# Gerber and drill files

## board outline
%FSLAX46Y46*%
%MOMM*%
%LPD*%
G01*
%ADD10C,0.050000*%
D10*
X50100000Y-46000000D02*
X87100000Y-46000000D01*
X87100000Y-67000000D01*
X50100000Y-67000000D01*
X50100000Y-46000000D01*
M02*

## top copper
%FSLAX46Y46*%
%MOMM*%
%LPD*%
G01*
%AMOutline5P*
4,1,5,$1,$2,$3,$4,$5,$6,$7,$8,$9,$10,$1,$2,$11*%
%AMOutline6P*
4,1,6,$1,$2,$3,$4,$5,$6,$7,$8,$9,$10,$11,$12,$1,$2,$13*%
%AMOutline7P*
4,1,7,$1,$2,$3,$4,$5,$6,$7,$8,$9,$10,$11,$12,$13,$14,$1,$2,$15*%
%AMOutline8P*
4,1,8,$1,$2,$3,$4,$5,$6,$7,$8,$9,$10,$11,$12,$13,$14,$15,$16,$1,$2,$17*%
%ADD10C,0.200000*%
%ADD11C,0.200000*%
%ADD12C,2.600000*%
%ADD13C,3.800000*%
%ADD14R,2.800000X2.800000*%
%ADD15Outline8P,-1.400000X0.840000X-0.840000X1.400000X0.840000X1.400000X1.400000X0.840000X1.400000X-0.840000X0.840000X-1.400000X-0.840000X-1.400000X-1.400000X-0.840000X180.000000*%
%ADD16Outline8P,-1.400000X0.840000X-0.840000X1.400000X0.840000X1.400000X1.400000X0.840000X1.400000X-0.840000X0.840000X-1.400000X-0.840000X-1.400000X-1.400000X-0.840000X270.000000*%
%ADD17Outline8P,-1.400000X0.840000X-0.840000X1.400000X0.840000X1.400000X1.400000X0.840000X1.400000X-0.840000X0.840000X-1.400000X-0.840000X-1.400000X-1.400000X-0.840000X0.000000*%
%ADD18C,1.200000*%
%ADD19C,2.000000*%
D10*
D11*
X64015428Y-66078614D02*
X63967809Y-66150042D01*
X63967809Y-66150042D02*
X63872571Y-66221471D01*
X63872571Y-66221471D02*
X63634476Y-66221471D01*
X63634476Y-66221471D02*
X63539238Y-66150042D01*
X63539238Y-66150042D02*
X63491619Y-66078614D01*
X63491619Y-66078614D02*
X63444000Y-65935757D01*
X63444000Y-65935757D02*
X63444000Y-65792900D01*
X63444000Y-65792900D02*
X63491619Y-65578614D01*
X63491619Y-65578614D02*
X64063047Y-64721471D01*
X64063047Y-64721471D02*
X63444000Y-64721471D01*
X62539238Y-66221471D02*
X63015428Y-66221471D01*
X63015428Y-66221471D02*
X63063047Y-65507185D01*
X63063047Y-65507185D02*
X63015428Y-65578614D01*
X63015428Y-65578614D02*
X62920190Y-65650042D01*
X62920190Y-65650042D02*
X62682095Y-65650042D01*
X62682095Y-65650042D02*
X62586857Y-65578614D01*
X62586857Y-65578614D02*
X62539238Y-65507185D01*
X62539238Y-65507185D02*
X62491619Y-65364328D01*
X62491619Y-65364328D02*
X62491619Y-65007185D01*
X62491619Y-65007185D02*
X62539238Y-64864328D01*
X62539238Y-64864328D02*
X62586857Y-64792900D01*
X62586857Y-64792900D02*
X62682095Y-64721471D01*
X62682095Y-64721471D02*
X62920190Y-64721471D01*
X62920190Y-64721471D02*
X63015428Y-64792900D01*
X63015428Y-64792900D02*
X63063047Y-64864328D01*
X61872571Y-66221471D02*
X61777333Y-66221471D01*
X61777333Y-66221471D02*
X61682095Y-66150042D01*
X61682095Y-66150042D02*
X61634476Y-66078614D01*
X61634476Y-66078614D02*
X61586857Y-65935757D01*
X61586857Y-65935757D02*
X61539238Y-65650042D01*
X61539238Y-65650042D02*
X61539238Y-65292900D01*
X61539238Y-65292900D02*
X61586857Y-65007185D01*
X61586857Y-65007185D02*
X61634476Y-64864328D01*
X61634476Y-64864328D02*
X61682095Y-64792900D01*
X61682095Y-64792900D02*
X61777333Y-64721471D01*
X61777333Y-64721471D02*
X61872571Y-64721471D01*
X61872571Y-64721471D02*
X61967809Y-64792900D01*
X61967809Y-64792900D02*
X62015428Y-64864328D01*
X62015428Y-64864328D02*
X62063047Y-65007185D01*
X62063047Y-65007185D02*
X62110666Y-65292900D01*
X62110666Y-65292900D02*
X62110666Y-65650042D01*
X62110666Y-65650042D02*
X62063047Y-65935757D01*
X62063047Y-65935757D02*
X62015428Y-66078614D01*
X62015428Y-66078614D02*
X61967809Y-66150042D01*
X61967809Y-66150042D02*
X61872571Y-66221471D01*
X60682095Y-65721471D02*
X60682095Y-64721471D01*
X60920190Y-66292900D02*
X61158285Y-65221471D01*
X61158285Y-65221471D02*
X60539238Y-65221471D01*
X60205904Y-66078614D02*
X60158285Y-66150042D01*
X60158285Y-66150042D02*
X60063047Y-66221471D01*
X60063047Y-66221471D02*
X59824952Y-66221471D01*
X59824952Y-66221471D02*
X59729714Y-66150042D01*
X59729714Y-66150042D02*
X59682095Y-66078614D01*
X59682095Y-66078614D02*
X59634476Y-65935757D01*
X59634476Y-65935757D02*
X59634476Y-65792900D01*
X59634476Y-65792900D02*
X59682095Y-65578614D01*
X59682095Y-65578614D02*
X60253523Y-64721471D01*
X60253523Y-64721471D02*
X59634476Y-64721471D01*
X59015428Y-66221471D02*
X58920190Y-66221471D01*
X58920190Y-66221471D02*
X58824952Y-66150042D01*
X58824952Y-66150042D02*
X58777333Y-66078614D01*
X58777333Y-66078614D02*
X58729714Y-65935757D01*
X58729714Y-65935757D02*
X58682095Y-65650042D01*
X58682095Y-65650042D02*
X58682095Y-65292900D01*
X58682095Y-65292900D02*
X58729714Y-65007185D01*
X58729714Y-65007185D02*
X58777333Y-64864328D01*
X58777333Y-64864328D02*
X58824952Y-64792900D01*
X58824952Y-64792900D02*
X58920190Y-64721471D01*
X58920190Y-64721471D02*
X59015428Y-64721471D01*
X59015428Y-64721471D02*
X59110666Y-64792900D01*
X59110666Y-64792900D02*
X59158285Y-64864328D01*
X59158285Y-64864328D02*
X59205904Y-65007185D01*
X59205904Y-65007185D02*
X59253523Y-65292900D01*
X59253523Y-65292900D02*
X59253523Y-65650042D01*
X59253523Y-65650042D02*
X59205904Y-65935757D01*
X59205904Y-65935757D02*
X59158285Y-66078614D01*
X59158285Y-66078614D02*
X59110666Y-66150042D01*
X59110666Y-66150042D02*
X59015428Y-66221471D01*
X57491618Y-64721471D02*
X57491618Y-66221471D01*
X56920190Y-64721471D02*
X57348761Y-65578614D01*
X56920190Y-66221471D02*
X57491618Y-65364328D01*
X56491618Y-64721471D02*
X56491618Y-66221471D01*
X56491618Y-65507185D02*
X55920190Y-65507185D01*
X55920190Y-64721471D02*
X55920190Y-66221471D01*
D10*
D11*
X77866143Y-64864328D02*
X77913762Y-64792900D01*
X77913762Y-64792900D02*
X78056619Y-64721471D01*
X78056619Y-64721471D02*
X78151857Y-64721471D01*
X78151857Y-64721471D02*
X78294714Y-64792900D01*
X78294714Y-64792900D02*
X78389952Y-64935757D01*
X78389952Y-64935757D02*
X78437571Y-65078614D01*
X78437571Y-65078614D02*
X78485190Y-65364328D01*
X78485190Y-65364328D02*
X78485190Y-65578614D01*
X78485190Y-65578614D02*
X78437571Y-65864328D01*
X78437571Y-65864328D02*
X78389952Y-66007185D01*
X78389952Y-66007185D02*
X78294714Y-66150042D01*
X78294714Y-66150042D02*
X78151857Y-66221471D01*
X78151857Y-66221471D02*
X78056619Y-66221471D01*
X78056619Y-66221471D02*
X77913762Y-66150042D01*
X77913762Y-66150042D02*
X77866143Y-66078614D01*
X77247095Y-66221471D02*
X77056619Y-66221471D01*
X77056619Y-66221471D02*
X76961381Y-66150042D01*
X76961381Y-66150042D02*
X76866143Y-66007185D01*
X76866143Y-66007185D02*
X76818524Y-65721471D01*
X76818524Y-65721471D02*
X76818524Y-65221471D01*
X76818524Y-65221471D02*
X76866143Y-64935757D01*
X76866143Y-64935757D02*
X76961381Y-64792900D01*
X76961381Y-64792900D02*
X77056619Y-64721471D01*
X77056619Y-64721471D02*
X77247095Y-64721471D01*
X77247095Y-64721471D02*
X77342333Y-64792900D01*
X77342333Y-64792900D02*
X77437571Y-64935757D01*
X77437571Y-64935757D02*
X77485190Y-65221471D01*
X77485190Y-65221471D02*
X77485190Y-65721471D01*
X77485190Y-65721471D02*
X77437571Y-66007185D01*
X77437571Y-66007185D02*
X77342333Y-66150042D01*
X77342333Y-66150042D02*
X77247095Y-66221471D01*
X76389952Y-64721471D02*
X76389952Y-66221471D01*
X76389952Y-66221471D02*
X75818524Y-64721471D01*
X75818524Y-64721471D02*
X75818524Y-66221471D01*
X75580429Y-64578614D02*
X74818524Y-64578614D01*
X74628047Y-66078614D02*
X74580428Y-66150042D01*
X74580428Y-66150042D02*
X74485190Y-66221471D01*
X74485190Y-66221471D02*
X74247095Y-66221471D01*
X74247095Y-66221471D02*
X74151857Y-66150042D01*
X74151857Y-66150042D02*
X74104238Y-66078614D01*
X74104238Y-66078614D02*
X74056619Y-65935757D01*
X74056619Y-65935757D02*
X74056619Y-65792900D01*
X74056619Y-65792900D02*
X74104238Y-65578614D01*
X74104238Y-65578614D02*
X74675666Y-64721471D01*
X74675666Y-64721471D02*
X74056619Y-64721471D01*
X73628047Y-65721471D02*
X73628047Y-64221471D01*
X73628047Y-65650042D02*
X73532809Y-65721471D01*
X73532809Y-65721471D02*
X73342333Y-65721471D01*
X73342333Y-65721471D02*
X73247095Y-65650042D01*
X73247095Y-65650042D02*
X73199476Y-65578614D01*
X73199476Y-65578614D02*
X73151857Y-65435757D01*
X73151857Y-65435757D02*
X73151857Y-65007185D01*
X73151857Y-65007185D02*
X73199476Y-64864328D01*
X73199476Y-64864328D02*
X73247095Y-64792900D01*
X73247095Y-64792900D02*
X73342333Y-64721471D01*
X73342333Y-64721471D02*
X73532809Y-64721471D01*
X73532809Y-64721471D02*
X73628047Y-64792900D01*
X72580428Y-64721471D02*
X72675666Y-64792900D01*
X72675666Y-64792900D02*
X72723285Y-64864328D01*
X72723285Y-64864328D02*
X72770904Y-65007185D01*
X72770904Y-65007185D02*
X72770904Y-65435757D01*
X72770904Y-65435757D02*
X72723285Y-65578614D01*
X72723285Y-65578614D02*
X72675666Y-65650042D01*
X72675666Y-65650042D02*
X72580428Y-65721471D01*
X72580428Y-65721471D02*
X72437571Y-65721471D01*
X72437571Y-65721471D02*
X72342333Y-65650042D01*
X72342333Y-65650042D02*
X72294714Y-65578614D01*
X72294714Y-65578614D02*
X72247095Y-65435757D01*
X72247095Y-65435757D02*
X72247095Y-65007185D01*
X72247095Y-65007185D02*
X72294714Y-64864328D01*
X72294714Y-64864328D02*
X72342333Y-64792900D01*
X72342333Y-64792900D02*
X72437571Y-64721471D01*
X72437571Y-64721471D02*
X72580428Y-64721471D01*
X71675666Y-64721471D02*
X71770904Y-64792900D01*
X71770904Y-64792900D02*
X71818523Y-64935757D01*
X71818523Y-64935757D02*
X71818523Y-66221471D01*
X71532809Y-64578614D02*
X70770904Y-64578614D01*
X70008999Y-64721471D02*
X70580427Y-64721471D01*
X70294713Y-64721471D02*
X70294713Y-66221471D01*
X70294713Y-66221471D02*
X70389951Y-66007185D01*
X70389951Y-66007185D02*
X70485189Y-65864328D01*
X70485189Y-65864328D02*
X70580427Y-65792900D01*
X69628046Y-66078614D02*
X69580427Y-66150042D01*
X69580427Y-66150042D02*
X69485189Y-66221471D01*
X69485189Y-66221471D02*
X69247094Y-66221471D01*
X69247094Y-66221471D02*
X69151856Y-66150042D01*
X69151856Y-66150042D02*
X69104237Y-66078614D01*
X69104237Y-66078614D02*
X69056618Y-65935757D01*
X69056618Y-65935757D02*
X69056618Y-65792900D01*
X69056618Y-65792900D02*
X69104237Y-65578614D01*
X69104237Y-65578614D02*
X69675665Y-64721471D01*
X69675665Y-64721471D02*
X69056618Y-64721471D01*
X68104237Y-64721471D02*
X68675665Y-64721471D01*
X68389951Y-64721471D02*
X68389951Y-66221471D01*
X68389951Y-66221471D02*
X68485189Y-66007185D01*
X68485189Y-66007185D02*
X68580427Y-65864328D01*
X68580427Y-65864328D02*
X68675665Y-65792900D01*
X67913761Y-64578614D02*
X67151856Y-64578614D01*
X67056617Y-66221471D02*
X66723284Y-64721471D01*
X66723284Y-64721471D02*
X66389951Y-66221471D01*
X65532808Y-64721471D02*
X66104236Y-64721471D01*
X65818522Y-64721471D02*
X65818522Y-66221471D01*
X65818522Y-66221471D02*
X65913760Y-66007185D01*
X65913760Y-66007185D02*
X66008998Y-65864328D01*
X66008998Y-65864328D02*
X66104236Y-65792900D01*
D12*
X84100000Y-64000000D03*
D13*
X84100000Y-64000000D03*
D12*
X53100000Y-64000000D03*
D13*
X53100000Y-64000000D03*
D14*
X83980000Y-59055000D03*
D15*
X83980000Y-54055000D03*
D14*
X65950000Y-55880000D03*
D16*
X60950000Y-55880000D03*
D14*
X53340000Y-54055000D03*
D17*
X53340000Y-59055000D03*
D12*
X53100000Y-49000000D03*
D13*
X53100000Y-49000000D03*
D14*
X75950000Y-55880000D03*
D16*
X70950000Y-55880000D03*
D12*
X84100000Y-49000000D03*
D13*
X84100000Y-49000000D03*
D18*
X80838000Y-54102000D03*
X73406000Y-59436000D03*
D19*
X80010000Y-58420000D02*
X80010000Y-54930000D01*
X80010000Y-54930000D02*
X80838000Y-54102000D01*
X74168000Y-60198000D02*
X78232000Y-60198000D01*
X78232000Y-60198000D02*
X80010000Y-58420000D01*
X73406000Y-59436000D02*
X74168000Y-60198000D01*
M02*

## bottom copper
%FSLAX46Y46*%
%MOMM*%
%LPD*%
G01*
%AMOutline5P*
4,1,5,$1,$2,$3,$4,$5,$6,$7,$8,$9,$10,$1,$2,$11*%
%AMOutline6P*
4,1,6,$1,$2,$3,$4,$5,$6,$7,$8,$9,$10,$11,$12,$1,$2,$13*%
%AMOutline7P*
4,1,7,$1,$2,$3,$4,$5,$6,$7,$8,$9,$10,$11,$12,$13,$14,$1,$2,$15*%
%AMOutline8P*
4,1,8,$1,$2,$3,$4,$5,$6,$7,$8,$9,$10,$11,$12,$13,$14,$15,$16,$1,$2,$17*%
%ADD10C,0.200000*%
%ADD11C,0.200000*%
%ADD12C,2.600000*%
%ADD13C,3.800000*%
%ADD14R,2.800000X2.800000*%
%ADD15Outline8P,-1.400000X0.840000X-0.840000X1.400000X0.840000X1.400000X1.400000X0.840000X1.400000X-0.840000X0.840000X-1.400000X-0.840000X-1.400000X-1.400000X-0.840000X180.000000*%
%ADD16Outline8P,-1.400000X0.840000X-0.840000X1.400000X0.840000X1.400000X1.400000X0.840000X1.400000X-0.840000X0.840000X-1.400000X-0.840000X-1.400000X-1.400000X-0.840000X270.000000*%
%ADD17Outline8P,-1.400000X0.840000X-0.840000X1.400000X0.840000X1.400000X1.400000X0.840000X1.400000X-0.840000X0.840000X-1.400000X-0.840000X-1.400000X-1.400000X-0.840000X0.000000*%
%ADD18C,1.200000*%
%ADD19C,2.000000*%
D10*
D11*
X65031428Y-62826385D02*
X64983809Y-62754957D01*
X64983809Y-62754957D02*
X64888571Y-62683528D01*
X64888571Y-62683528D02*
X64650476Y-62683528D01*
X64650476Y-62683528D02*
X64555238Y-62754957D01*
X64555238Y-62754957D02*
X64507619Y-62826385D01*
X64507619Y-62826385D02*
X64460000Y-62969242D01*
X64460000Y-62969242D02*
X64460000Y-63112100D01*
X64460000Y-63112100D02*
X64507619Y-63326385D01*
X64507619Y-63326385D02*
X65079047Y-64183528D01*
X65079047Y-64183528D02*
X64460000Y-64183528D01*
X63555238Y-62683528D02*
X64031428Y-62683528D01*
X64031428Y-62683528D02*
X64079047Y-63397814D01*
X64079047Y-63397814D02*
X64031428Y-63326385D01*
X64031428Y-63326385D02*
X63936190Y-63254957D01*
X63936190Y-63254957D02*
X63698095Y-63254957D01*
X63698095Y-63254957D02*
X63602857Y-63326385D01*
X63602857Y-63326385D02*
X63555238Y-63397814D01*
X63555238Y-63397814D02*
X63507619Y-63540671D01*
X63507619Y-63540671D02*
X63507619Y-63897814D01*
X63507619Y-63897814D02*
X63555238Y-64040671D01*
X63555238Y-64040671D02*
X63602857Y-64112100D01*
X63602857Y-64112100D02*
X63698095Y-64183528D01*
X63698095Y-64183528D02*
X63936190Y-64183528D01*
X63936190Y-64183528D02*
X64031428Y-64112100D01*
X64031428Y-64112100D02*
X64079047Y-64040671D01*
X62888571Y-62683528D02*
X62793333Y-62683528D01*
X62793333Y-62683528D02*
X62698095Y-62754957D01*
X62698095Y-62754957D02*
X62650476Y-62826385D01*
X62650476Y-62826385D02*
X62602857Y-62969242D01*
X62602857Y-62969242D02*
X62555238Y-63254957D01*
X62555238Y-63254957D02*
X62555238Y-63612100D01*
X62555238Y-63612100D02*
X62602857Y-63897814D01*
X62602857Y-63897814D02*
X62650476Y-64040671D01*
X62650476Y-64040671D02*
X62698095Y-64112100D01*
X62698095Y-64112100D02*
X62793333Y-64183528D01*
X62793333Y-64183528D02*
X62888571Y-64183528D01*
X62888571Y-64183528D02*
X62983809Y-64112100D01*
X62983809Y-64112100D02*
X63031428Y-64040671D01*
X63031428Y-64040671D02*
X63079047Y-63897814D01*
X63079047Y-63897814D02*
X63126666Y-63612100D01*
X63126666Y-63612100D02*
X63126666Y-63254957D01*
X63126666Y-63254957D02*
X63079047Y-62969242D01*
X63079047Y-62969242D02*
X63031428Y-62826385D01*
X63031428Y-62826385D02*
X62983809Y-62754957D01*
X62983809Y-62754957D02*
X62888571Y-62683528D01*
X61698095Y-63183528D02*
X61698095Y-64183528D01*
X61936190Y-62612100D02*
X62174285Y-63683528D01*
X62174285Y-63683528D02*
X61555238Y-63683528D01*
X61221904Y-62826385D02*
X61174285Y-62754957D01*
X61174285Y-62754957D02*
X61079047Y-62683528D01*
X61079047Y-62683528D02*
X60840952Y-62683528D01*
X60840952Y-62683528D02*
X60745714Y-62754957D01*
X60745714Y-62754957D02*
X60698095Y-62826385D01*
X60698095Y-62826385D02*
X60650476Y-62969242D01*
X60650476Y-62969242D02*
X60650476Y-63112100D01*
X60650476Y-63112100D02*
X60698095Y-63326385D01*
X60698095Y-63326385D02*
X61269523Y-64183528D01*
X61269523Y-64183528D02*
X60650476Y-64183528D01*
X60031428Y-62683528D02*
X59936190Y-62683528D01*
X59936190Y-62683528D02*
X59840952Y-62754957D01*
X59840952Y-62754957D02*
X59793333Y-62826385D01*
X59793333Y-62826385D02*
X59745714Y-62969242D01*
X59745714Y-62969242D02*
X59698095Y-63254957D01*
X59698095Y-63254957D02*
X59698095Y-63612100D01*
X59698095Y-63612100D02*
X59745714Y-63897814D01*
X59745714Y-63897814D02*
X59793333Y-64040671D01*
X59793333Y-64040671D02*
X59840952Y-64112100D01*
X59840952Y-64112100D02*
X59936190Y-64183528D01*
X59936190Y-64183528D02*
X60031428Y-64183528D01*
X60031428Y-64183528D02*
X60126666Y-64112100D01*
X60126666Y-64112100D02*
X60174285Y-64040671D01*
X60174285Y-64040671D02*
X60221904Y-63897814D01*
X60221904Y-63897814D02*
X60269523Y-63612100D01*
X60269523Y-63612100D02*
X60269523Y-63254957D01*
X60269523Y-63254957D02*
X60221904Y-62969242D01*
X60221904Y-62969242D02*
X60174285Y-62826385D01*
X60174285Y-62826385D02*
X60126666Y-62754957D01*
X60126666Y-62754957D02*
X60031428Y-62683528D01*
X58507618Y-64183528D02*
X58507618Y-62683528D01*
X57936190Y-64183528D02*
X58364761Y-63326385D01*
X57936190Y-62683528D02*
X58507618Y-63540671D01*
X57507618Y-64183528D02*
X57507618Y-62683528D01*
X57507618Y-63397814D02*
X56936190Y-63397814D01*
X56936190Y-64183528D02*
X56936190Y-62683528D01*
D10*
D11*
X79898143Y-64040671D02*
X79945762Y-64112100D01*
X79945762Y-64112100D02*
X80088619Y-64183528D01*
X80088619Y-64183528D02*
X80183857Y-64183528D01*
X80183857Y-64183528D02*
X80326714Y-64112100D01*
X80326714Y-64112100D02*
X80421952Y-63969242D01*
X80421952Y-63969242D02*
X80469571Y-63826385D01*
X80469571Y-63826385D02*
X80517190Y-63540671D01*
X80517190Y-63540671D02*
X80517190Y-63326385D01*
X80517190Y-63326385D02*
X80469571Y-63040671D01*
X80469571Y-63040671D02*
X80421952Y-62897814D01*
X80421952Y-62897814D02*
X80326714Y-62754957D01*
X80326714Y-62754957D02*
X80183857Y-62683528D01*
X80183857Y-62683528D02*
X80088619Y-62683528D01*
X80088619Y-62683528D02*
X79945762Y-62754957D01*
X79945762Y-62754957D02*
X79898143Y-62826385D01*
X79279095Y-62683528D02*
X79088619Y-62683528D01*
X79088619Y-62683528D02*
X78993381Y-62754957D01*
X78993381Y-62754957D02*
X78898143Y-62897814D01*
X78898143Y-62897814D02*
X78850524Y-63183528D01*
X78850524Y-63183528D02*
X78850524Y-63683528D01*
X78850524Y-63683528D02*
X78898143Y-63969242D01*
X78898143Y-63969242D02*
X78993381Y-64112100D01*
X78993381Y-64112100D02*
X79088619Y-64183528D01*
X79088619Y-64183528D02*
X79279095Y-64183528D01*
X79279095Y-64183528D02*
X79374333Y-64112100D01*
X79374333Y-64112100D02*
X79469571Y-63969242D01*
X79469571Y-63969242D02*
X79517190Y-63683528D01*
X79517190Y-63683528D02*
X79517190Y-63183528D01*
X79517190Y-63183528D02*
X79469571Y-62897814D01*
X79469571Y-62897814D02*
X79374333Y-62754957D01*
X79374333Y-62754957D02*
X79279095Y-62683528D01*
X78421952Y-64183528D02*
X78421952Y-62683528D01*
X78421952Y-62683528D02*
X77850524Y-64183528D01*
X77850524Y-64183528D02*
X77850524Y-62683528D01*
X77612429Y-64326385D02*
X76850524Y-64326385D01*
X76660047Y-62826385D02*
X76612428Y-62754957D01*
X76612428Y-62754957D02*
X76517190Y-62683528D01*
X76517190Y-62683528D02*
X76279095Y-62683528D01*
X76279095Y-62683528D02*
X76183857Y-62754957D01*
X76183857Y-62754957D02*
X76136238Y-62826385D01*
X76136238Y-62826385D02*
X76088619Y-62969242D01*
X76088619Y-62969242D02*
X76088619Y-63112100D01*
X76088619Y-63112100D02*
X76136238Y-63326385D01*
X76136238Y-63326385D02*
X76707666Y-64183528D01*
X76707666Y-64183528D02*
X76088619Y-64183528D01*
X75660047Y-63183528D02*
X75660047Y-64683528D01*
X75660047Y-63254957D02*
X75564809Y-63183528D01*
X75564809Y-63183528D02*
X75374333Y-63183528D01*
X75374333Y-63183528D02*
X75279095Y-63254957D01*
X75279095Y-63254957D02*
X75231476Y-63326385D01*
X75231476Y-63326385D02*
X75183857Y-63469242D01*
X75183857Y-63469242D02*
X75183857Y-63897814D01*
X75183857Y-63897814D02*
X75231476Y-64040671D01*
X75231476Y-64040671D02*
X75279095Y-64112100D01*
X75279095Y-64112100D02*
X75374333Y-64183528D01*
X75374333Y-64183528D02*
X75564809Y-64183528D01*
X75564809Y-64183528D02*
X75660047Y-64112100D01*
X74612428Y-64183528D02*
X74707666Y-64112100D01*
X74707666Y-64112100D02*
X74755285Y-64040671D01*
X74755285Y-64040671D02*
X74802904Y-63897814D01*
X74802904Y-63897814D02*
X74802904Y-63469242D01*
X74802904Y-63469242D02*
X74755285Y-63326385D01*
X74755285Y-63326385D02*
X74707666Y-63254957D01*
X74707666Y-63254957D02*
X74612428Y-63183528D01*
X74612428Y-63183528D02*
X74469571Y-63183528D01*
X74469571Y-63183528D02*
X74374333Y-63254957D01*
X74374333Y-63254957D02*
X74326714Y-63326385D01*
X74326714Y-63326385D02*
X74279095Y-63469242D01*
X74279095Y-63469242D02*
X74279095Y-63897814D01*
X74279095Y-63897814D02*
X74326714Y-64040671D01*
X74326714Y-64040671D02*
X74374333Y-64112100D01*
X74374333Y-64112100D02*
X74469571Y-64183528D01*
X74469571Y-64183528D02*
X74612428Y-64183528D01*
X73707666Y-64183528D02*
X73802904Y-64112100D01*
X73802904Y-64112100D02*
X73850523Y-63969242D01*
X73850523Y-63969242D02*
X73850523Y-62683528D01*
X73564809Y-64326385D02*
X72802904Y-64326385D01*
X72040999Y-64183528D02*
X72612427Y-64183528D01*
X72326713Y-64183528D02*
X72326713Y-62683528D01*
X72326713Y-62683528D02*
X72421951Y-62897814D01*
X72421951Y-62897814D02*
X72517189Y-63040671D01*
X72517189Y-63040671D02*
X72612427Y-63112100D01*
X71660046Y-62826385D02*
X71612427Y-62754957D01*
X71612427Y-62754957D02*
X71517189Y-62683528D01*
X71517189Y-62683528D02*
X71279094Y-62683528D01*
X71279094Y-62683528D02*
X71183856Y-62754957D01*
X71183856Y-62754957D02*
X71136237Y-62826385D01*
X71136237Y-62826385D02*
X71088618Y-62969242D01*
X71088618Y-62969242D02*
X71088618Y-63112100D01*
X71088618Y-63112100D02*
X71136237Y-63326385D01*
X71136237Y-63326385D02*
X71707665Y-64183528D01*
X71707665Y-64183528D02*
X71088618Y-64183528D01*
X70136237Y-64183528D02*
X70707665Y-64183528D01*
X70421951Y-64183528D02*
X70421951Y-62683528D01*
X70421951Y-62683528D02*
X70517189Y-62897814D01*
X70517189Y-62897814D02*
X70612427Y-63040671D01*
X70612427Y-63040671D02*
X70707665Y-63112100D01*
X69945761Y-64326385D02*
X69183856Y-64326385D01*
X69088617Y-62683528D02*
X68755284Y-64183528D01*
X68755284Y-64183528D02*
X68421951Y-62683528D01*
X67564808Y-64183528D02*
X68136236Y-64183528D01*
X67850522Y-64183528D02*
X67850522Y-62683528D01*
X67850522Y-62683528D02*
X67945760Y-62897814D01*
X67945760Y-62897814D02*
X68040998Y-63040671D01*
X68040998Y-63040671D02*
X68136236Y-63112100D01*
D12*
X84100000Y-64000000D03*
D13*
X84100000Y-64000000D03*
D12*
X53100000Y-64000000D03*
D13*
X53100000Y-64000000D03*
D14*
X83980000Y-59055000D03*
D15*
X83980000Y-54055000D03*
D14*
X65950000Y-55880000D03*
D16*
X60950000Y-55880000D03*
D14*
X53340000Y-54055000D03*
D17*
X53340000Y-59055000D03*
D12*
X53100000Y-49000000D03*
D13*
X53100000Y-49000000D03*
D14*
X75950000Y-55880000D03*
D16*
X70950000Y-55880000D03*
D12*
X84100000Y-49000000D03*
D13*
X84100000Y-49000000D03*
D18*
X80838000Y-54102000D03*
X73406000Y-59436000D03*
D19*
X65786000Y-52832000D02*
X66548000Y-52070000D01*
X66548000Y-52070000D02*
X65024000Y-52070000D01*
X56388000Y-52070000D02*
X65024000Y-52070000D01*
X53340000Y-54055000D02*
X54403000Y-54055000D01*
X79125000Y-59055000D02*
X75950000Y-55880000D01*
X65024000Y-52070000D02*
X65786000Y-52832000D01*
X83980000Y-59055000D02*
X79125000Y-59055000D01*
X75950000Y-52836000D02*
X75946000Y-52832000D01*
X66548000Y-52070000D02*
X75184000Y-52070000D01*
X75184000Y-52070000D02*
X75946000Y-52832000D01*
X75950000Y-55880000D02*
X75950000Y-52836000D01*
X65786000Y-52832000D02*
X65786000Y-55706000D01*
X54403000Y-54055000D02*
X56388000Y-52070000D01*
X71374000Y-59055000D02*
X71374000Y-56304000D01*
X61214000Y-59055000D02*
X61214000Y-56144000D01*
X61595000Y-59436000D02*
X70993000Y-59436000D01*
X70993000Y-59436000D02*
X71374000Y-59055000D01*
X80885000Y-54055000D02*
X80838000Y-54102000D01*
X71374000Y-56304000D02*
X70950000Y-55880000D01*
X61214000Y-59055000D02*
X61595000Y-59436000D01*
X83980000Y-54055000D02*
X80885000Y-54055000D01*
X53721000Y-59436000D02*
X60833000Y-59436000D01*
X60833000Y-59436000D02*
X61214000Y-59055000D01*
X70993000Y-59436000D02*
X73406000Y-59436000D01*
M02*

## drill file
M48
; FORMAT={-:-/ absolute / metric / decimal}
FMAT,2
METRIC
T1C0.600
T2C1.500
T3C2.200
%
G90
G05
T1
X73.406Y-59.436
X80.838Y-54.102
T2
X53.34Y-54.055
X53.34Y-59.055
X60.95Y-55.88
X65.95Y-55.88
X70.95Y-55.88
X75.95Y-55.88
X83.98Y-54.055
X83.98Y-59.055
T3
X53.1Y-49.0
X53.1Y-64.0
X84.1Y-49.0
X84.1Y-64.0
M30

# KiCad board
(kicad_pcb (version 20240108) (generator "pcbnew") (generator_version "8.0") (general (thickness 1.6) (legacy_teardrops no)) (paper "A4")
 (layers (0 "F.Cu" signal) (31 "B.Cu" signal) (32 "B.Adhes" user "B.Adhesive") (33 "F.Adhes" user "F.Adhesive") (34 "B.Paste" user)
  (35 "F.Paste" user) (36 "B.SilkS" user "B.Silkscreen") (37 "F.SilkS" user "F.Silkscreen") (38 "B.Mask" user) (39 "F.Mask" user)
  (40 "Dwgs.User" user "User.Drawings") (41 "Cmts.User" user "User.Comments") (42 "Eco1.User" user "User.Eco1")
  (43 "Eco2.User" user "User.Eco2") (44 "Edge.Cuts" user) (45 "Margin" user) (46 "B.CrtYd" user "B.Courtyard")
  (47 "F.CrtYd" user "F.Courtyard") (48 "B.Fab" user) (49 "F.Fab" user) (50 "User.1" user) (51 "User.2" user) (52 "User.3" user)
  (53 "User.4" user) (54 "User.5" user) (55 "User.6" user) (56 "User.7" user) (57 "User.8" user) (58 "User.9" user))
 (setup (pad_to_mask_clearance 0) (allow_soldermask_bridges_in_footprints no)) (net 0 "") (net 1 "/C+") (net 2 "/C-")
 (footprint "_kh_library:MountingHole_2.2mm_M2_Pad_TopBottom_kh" (layer "F.Cu") (at 84.1 64)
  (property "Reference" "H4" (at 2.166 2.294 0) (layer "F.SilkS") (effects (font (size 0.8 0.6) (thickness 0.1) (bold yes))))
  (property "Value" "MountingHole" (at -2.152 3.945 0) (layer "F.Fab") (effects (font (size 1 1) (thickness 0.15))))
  (pad "1" thru_hole circle (at 0 0) (size 2.6 2.6) (drill 2.2) (layers "*.Cu" "*.Mask") (remove_unused_layers no))
  (pad "1" connect circle (at 0 0) (size 3.8 3.8) (layers "F.Cu" "F.Mask"))
  (pad "1" connect circle (at 0 0) (size 3.8 3.8) (layers "B.Cu" "B.Mask")))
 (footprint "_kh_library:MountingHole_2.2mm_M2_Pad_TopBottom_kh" (layer "F.Cu") (at 53.1 64)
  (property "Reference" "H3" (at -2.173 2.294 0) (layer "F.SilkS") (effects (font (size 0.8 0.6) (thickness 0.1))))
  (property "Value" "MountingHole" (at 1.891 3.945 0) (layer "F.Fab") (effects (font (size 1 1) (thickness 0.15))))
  (pad "1" thru_hole circle (at 0 0) (size 2.6 2.6) (drill 2.2) (layers "*.Cu" "*.Mask") (remove_unused_layers no))
  (pad "1" connect circle (at 0 0) (size 3.8 3.8) (layers "F.Cu" "F.Mask"))
  (pad "1" connect circle (at 0 0) (size 3.8 3.8) (layers "B.Cu" "B.Mask")))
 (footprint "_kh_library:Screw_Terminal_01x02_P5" (layer "F.Cu") (at 83.98 59.055 180)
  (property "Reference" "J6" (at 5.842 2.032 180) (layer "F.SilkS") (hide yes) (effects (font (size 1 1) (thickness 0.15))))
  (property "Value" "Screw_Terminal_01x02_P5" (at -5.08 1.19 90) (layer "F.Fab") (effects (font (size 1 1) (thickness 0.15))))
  (pad "1" thru_hole rect (at 0 0 180) (size 2.8 2.8) (drill 1.5) (layers "*.Cu" "*.Mask") (remove_unused_layers no) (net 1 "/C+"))
  (pad "2" thru_hole roundrect (at 0 5 180) (size 2.8 2.8) (drill 1.5) (layers "*.Cu" "*.Mask") (remove_unused_layers no)
   (roundrect_rratio 0) (chamfer_ratio 0.2) (chamfer top_left top_right bottom_left bottom_right) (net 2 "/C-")))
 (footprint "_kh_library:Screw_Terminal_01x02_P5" (layer "F.Cu") (at 65.95 55.88 -90)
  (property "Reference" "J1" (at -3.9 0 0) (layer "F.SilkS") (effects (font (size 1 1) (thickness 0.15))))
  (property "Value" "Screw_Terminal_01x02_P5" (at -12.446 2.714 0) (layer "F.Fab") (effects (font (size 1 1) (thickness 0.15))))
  (pad "1" thru_hole rect (at 0 0 270) (size 2.8 2.8) (drill 1.5) (layers "*.Cu" "*.Mask") (remove_unused_layers no) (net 1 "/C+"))
  (pad "2" thru_hole roundrect (at 0 5 270) (size 2.8 2.8) (drill 1.5) (layers "*.Cu" "*.Mask") (remove_unused_layers no)
   (roundrect_rratio 0) (chamfer_ratio 0.2) (chamfer top_left top_right bottom_left bottom_right) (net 2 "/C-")))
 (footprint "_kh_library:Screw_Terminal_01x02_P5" (layer "F.Cu") (at 53.34 54.055)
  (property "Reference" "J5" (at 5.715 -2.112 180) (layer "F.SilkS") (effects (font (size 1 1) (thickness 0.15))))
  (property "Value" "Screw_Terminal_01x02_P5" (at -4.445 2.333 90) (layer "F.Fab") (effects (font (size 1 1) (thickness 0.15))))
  (pad "1" thru_hole rect (at 0 0) (size 2.8 2.8) (drill 1.5) (layers "*.Cu" "*.Mask") (remove_unused_layers no) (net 1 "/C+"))
  (pad "2" thru_hole roundrect (at 0 5) (size 2.8 2.8) (drill 1.5) (layers "*.Cu" "*.Mask") (remove_unused_layers no) (roundrect_rratio 0)
   (chamfer_ratio 0.2) (chamfer top_left top_right bottom_left bottom_right) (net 2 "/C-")))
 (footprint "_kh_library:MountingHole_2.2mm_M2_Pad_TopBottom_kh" (layer "F.Cu") (at 53.1 49)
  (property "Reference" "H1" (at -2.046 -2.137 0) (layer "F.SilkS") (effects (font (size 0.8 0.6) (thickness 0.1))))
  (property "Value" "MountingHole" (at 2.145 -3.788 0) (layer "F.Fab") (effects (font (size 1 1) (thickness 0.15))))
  (pad "1" thru_hole circle (at 0 0) (size 2.6 2.6) (drill 2.2) (layers "*.Cu" "*.Mask") (remove_unused_layers no))
  (pad "1" connect circle (at 0 0) (size 3.8 3.8) (layers "F.Cu" "F.Mask"))
  (pad "1" connect circle (at 0 0) (size 3.8 3.8) (layers "B.Cu" "B.Mask")))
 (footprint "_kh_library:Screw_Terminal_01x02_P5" (layer "F.Cu") (at 75.95 55.88 -90)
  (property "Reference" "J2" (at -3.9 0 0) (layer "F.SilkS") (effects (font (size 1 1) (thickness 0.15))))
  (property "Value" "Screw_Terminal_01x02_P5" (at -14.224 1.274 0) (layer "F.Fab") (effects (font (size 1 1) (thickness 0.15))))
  (pad "1" thru_hole rect (at 0 0 270) (size 2.8 2.8) (drill 1.5) (layers "*.Cu" "*.Mask") (remove_unused_layers no) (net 1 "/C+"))
  (pad "2" thru_hole roundrect (at 0 5 270) (size 2.8 2.8) (drill 1.5) (layers "*.Cu" "*.Mask") (remove_unused_layers no)
   (roundrect_rratio 0) (chamfer_ratio 0.2) (chamfer top_left top_right bottom_left bottom_right) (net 2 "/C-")))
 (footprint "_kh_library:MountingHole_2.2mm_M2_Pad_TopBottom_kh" (layer "F.Cu") (at 84.1 49)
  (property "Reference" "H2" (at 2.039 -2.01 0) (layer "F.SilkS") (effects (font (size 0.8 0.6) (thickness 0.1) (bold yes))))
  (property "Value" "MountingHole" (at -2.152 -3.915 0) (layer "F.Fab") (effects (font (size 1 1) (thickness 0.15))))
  (pad "1" thru_hole circle (at 0 0) (size 2.6 2.6) (drill 2.2) (layers "*.Cu" "*.Mask") (remove_unused_layers no))
  (pad "1" connect circle (at 0 0) (size 3.8 3.8) (layers "F.Cu" "F.Mask"))
  (pad "1" connect circle (at 0 0) (size 3.8 3.8) (layers "B.Cu" "B.Mask")))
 (gr_rect (start 50.1 46) (end 87.1 67) (stroke (width 0.05) (type default)) (fill none) (layer "Edge.Cuts"))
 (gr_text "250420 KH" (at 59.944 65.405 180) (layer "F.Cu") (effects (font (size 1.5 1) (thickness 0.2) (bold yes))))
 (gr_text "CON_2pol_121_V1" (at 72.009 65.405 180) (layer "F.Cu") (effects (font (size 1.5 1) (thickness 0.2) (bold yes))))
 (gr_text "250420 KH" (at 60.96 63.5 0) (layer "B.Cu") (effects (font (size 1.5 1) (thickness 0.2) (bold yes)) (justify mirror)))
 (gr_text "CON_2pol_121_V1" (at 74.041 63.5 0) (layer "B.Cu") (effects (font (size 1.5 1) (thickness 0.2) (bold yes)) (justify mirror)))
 (segment (start 65.786 52.832) (end 66.548 52.07) (width 2) (layer "B.Cu") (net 1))
 (segment (start 66.548 52.07) (end 65.024 52.07) (width 2) (layer "B.Cu") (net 1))
 (segment (start 56.388 52.07) (end 65.024 52.07) (width 2) (layer "B.Cu") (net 1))
 (segment (start 53.34 54.055) (end 54.403 54.055) (width 2) (layer "B.Cu") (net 1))
 (segment (start 79.125 59.055) (end 75.95 55.88) (width 2) (layer "B.Cu") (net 1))
 (segment (start 65.024 52.07) (end 65.786 52.832) (width 2) (layer "B.Cu") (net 1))
 (segment (start 83.98 59.055) (end 79.125 59.055) (width 2) (layer "B.Cu") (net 1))
 (segment (start 75.95 52.836) (end 75.946 52.832) (width 2) (layer "B.Cu") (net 1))
 (segment (start 66.548 52.07) (end 75.184 52.07) (width 2) (layer "B.Cu") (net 1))
 (segment (start 75.184 52.07) (end 75.946 52.832) (width 2) (layer "B.Cu") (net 1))
 (segment (start 75.95 55.88) (end 75.95 52.836) (width 2) (layer "B.Cu") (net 1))
 (segment (start 65.786 52.832) (end 65.786 55.706) (width 2) (layer "B.Cu") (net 1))
 (segment (start 54.403 54.055) (end 56.388 52.07) (width 2) (layer "B.Cu") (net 1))
 (segment (start 80.01 58.42) (end 80.01 54.93) (width 2) (layer "F.Cu") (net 2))
 (segment (start 80.01 54.93) (end 80.838 54.102) (width 2) (layer "F.Cu") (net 2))
 (segment (start 74.168 60.198) (end 78.232 60.198) (width 2) (layer "F.Cu") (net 2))
 (segment (start 78.232 60.198) (end 80.01 58.42) (width 2) (layer "F.Cu") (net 2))
 (segment (start 73.406 59.436) (end 74.168 60.198) (width 2) (layer "F.Cu") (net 2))
 (via (at 80.838 54.102) (size 1.2) (drill 0.6) (layers "F.Cu" "B.Cu") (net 2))
 (via (at 73.406 59.436) (size 1.2) (drill 0.6) (layers "F.Cu" "B.Cu") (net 2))
 (segment (start 71.374 59.055) (end 71.374 56.304) (width 2) (layer "B.Cu") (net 2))
 (segment (start 61.214 59.055) (end 61.214 56.144) (width 2) (layer "B.Cu") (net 2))
 (segment (start 61.595 59.436) (end 70.993 59.436) (width 2) (layer "B.Cu") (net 2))
 (segment (start 70.993 59.436) (end 71.374 59.055) (width 2) (layer "B.Cu") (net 2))
 (segment (start 80.885 54.055) (end 80.838 54.102) (width 2) (layer "B.Cu") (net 2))
 (segment (start 71.374 56.304) (end 70.95 55.88) (width 2) (layer "B.Cu") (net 2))
 (segment (start 61.214 59.055) (end 61.595 59.436) (width 2) (layer "B.Cu") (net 2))
 (segment (start 83.98 54.055) (end 80.885 54.055) (width 2) (layer "B.Cu") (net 2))
 (segment (start 53.721 59.436) (end 60.833 59.436) (width 2) (layer "B.Cu") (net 2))
 (segment (start 60.833 59.436) (end 61.214 59.055) (width 2) (layer "B.Cu") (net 2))
 (segment (start 70.993 59.436) (end 73.406 59.436) (width 2) (layer "B.Cu") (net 2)))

